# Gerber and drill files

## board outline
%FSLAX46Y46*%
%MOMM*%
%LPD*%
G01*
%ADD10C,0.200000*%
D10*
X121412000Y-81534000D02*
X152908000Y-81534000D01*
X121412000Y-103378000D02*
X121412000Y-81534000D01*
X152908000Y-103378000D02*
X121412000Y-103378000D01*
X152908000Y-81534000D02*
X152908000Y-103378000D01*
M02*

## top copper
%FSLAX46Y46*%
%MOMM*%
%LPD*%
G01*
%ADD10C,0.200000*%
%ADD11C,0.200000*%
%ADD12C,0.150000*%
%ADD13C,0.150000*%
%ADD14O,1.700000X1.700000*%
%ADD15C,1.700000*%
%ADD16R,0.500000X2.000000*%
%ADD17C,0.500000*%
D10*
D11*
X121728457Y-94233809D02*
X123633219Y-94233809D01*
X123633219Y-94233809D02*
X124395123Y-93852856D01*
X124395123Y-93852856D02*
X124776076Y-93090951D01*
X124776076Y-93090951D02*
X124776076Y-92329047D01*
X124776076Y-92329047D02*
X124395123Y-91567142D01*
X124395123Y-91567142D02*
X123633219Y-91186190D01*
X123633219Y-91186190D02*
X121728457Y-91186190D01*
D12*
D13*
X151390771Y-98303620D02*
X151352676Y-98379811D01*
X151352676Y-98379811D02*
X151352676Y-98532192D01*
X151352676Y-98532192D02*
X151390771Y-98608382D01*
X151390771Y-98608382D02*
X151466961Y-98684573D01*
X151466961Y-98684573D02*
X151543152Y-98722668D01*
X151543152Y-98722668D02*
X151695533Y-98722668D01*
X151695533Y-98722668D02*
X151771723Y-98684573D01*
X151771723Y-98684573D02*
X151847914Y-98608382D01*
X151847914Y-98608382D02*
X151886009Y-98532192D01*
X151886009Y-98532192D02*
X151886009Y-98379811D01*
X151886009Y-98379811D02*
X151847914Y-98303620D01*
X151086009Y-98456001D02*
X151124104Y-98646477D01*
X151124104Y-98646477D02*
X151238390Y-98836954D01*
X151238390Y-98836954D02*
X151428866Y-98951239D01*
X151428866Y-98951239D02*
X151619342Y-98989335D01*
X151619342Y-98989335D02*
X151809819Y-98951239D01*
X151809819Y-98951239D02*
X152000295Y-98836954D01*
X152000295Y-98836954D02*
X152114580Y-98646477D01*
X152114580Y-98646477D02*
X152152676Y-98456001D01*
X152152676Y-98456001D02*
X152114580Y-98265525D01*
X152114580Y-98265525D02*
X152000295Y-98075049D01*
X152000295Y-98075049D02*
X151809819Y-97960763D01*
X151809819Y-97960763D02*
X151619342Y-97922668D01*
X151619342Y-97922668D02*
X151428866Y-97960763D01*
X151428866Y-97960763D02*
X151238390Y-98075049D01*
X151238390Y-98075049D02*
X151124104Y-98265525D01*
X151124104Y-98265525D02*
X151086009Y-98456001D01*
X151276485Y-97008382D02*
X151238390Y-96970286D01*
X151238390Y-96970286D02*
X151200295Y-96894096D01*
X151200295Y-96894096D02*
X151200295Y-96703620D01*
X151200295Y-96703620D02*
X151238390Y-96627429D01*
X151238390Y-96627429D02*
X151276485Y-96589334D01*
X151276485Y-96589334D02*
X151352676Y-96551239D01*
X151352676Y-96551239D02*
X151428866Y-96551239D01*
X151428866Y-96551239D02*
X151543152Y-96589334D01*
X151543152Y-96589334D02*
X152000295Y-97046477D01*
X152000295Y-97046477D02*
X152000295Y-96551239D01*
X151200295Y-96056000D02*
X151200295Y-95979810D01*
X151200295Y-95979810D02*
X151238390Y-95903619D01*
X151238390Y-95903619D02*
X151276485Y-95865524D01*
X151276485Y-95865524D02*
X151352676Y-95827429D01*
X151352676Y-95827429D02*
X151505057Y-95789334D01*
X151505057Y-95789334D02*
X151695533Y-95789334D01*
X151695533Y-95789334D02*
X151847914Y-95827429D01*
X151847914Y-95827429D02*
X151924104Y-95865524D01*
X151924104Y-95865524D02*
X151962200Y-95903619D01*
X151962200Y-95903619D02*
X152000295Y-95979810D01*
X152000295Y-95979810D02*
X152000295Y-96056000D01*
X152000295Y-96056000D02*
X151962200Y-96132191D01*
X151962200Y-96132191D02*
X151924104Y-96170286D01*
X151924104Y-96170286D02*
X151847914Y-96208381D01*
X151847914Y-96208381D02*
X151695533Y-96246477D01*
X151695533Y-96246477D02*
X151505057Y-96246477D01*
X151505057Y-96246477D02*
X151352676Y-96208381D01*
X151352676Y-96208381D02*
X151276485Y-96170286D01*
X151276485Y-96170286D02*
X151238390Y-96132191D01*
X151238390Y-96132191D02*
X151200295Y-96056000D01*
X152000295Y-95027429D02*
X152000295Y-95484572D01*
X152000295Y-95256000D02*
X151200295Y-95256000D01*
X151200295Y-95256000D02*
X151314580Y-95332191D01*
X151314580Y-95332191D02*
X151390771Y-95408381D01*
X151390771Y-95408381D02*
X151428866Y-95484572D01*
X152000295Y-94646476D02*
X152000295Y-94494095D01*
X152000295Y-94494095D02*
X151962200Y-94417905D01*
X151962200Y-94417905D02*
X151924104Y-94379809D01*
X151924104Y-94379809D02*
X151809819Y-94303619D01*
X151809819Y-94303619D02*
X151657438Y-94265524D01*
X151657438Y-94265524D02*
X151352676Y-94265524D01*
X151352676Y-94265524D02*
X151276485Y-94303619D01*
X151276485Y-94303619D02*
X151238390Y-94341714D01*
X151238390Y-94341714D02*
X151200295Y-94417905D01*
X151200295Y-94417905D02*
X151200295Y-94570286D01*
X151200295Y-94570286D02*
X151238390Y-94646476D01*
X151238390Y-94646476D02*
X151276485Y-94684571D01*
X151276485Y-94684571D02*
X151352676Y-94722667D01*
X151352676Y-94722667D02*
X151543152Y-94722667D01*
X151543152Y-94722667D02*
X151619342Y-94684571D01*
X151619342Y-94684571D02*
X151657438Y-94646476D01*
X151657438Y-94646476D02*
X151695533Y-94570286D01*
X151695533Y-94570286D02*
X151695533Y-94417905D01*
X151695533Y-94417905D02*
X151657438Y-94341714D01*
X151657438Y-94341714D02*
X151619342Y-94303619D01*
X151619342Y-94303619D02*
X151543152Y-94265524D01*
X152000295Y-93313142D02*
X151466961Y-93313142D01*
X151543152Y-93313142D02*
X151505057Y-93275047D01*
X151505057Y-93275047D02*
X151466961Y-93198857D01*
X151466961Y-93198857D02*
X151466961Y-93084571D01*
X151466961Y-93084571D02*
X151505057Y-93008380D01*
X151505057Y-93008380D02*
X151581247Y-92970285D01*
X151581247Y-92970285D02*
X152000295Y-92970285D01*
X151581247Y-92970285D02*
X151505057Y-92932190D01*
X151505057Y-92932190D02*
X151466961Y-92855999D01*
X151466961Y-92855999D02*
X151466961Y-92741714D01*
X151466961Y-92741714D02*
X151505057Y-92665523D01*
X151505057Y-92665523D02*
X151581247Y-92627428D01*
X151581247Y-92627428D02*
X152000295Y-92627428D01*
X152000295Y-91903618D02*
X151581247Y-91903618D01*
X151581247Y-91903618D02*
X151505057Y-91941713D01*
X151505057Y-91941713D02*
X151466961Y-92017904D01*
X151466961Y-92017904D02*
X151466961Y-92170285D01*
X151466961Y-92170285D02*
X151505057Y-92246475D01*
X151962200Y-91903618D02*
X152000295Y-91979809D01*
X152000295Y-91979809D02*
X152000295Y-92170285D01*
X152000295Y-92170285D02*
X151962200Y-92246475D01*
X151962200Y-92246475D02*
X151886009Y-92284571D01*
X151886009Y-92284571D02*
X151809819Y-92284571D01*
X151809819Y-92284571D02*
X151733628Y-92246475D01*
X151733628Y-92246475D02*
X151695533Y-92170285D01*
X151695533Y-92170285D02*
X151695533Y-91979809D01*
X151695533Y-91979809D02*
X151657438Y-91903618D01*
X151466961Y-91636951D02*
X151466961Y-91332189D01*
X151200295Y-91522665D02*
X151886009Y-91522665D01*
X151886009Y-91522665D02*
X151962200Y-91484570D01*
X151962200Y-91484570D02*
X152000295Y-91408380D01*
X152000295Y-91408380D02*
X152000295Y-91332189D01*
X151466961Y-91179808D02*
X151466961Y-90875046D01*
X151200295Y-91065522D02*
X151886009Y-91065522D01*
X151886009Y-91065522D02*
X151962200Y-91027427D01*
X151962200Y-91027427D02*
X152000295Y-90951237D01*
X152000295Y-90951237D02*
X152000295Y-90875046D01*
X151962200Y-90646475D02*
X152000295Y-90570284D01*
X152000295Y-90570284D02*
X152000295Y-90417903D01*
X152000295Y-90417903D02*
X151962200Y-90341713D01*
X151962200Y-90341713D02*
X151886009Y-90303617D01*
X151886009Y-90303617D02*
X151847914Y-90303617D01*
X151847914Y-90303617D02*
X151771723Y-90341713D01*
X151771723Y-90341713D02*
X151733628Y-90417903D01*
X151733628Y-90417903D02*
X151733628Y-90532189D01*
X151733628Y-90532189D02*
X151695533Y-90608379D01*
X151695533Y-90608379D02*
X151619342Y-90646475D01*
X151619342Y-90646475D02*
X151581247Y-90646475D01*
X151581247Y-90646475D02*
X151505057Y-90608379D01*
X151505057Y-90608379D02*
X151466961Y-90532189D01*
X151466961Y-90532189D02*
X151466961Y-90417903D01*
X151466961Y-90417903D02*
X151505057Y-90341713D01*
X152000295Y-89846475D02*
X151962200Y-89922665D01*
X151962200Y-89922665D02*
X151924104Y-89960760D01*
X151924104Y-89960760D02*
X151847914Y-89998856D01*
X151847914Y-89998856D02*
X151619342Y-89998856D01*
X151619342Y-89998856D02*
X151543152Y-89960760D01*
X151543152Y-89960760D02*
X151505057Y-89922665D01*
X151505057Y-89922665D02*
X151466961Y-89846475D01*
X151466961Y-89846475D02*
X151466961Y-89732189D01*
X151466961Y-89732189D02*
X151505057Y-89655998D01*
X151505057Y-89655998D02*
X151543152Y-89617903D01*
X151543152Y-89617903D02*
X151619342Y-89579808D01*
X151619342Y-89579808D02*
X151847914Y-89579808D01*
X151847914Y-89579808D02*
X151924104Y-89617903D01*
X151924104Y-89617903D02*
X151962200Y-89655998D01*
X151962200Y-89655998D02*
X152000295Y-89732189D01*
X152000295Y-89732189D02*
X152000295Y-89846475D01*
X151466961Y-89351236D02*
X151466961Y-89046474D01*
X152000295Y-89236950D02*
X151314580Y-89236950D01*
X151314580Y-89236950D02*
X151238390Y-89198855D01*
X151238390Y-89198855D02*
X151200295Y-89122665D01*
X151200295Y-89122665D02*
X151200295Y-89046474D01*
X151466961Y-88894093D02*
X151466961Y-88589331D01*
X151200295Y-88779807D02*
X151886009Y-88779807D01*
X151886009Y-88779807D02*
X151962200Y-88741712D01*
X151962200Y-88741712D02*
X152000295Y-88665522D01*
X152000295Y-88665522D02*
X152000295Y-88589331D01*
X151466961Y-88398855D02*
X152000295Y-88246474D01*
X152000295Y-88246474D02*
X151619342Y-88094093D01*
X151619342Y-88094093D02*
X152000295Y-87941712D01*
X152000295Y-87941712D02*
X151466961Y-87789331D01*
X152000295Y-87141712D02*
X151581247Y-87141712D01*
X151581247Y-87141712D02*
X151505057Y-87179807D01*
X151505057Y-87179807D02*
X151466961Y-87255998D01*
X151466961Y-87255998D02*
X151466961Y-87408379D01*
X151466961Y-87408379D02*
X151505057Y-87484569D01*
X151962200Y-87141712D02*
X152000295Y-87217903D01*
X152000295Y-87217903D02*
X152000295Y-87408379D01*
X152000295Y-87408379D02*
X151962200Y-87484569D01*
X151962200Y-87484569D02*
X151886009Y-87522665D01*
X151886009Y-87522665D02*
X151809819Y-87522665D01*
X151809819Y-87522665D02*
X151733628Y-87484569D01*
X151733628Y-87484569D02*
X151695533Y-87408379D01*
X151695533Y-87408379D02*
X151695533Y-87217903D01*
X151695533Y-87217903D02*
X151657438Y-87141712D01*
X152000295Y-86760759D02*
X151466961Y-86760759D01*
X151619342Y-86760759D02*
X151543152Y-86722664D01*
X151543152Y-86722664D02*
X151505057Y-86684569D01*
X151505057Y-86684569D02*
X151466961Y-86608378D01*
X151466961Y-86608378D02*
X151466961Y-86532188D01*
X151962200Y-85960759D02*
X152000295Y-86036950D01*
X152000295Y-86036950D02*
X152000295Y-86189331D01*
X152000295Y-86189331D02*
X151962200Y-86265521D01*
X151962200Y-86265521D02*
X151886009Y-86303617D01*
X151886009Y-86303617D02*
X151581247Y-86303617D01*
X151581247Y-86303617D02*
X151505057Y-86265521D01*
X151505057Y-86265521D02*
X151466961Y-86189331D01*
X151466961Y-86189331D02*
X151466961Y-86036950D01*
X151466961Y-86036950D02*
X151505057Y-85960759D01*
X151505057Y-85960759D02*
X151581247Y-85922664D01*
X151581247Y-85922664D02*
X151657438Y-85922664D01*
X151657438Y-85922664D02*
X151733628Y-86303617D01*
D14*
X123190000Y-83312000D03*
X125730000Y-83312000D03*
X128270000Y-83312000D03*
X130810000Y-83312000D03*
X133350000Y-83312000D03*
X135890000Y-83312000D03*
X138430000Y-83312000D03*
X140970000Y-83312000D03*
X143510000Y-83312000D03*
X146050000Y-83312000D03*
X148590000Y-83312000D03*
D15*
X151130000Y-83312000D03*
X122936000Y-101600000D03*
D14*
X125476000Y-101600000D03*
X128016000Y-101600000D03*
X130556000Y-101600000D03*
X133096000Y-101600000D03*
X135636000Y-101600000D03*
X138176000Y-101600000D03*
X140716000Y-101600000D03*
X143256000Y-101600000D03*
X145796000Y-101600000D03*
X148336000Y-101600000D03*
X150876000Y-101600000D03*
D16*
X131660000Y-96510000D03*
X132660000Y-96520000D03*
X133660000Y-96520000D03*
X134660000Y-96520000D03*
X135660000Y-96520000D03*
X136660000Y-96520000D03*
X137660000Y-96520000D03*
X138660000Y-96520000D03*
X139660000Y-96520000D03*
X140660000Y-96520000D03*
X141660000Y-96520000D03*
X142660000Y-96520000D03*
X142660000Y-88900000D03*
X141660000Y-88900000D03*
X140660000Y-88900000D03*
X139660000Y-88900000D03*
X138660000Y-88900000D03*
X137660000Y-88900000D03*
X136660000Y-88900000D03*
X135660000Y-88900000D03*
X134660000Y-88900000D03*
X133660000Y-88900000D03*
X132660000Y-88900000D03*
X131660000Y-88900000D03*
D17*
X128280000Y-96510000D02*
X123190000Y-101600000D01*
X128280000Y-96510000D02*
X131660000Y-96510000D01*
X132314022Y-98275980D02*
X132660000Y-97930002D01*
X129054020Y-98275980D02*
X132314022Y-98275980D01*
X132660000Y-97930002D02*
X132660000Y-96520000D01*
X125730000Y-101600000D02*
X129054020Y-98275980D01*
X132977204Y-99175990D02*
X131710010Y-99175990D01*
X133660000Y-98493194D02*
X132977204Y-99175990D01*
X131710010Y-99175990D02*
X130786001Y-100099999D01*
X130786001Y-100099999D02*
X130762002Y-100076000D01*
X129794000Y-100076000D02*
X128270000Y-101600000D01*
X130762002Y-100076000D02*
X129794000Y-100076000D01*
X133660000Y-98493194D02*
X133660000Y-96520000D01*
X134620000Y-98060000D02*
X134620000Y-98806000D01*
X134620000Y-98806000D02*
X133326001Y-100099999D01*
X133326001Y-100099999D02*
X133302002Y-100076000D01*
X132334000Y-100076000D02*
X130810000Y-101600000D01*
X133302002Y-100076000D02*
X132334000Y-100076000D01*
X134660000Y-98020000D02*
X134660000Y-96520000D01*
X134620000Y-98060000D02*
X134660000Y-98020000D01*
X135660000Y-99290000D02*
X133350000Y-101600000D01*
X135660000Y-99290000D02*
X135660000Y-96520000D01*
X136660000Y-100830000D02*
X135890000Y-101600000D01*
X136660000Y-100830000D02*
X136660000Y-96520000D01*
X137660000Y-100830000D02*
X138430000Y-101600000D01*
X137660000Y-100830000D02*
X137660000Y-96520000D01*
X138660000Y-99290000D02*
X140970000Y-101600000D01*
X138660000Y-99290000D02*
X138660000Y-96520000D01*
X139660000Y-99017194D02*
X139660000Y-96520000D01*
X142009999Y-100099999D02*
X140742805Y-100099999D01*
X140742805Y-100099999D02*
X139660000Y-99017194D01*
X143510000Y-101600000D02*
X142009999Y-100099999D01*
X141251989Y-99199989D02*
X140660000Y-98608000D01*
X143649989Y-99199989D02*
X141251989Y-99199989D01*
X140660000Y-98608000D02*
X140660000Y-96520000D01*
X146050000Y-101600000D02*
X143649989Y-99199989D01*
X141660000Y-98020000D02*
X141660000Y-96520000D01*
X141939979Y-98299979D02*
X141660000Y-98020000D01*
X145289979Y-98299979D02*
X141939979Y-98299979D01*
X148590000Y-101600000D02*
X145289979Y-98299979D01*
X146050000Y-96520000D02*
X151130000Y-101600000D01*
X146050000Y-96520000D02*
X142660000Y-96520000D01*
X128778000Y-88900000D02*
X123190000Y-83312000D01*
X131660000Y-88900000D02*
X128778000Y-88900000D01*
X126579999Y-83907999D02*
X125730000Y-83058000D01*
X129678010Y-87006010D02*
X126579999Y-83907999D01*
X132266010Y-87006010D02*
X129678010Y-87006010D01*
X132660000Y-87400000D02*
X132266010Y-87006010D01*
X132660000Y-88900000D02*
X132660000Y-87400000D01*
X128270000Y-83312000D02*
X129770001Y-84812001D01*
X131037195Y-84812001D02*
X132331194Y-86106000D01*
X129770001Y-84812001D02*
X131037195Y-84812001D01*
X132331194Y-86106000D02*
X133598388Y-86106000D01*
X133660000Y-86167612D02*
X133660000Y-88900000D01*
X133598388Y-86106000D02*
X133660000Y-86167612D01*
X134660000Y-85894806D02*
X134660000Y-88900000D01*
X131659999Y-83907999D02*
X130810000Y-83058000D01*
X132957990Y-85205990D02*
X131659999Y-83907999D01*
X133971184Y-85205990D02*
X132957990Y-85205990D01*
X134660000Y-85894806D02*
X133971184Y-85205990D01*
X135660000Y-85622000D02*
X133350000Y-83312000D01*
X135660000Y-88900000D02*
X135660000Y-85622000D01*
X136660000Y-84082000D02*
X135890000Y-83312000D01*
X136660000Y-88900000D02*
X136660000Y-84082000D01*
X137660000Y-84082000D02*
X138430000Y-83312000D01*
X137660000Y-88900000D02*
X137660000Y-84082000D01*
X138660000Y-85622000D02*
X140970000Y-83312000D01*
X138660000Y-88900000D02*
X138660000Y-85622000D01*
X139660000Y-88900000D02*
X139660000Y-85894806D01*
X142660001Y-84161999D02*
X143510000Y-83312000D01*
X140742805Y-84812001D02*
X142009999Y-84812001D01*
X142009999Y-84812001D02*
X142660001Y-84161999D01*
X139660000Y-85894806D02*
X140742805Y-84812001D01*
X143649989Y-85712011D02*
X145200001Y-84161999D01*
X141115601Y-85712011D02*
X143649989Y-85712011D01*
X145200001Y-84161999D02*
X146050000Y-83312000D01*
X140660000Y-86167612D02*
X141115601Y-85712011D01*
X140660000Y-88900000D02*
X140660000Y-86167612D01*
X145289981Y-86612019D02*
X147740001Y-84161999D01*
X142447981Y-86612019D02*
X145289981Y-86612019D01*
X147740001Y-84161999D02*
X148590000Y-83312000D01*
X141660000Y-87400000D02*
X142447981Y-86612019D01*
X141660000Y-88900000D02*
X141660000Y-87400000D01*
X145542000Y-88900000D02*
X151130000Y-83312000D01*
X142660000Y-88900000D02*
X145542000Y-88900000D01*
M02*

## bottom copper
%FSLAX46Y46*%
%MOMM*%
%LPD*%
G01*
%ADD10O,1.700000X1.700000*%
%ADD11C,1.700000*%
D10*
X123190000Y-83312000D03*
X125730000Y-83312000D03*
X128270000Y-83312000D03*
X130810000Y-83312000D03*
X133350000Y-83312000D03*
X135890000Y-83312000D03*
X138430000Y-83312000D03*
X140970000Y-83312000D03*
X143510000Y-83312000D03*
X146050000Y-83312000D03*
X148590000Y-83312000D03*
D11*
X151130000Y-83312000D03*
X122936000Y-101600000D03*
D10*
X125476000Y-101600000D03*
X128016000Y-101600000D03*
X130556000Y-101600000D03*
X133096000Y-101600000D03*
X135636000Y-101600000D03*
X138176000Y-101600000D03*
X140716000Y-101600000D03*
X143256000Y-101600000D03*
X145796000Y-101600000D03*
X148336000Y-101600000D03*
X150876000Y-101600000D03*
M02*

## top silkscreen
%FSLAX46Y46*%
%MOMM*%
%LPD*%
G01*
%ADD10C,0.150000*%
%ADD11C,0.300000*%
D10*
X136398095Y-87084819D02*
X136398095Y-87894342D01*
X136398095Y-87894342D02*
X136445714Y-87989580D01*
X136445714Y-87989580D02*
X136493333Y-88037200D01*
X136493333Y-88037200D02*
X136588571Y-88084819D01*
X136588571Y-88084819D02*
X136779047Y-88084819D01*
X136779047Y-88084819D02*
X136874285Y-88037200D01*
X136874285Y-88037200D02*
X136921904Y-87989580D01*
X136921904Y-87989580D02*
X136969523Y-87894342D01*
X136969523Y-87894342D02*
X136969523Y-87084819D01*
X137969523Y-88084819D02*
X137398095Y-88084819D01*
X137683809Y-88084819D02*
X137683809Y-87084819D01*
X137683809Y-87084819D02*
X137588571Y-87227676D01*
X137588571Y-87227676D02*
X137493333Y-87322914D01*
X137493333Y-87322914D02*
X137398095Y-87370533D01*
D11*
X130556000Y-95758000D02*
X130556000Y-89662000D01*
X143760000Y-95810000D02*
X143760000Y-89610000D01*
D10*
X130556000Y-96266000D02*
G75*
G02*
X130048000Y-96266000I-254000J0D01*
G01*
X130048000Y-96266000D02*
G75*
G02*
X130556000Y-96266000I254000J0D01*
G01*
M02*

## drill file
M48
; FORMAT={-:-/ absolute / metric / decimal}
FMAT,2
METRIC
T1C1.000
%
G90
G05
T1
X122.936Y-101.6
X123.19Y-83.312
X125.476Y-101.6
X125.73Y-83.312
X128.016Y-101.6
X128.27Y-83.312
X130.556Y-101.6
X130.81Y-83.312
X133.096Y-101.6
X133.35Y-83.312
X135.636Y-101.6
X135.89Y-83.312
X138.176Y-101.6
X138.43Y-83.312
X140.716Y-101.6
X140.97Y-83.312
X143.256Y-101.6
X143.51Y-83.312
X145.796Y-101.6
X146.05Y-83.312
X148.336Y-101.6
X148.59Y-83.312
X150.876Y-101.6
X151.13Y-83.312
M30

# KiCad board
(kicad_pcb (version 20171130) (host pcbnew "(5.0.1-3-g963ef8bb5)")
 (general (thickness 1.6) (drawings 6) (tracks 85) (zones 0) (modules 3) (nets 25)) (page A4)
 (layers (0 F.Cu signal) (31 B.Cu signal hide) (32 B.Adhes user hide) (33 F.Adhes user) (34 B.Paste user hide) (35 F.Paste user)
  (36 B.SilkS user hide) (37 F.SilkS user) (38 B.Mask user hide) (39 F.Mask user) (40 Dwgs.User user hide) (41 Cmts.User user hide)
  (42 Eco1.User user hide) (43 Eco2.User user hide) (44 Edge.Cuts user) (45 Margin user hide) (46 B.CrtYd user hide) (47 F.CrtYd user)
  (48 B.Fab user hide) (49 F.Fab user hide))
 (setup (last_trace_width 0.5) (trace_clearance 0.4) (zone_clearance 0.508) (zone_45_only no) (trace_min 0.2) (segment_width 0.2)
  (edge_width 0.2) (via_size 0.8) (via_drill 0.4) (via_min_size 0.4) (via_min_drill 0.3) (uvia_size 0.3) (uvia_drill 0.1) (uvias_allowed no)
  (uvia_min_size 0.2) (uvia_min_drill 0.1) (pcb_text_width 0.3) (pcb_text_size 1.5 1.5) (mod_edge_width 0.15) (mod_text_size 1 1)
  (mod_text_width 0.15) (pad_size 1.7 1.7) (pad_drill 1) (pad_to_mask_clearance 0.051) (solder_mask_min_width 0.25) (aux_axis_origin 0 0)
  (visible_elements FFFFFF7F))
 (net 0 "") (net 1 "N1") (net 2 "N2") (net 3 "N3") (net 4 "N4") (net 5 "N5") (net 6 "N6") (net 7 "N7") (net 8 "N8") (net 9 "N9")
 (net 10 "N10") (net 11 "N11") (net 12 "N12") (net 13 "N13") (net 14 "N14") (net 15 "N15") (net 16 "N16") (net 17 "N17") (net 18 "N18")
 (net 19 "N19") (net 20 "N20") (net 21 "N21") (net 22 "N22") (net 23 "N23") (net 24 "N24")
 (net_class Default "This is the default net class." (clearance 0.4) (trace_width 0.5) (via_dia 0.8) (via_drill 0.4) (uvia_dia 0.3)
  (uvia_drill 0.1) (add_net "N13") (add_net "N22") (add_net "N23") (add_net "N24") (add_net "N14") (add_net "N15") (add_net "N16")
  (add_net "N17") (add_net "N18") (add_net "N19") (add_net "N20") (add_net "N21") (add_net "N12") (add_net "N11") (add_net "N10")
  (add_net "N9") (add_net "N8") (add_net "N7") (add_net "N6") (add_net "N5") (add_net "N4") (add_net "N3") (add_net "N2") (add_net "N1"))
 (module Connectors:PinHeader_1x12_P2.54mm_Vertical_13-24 (layer B.Cu) (at 151.13 83.312 90)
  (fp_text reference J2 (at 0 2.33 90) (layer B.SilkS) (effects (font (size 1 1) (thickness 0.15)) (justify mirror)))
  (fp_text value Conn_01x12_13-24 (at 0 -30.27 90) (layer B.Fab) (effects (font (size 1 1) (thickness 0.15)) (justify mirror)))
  (pad 24 thru_hole oval (at 0 -27.94 90) (size 1.7 1.7) (drill 1) (layers *.Cu *.Mask) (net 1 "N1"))
  (pad 23 thru_hole oval (at 0 -25.4 90) (size 1.7 1.7) (drill 1) (layers *.Cu *.Mask) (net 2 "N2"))
  (pad 22 thru_hole oval (at 0 -22.86 90) (size 1.7 1.7) (drill 1) (layers *.Cu *.Mask) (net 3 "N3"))
  (pad 21 thru_hole oval (at 0 -20.32 90) (size 1.7 1.7) (drill 1) (layers *.Cu *.Mask) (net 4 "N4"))
  (pad 20 thru_hole oval (at 0 -17.78 90) (size 1.7 1.7) (drill 1) (layers *.Cu *.Mask) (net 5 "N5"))
  (pad 19 thru_hole oval (at 0 -15.24 90) (size 1.7 1.7) (drill 1) (layers *.Cu *.Mask) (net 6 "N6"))
  (pad 18 thru_hole oval (at 0 -12.7 90) (size 1.7 1.7) (drill 1) (layers *.Cu *.Mask) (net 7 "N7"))
  (pad 17 thru_hole oval (at 0 -10.16 90) (size 1.7 1.7) (drill 1) (layers *.Cu *.Mask) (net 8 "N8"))
  (pad 16 thru_hole oval (at 0 -7.62 90) (size 1.7 1.7) (drill 1) (layers *.Cu *.Mask) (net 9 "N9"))
  (pad 15 thru_hole oval (at 0 -5.08 90) (size 1.7 1.7) (drill 1) (layers *.Cu *.Mask) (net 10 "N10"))
  (pad 14 thru_hole oval (at 0 -2.54 90) (size 1.7 1.7) (drill 1) (layers *.Cu *.Mask) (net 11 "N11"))
  (pad 13 thru_hole circle (at 0 0 90) (size 1.7 1.7) (drill 1) (layers *.Cu *.Mask) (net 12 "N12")))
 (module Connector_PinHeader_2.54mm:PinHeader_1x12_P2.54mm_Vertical (layer B.Cu) (at 122.936 101.6 270)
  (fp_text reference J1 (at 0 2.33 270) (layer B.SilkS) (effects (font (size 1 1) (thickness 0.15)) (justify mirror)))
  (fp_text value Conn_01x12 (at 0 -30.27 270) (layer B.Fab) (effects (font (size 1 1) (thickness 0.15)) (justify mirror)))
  (pad 1 thru_hole circle (at 0 0 270) (size 1.7 1.7) (drill 1) (layers *.Cu *.Mask) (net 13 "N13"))
  (pad 2 thru_hole oval (at 0 -2.54 270) (size 1.7 1.7) (drill 1) (layers *.Cu *.Mask) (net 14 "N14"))
  (pad 3 thru_hole oval (at 0 -5.08 270) (size 1.7 1.7) (drill 1) (layers *.Cu *.Mask) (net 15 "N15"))
  (pad 4 thru_hole oval (at 0 -7.62 270) (size 1.7 1.7) (drill 1) (layers *.Cu *.Mask) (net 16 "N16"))
  (pad 5 thru_hole oval (at 0 -10.16 270) (size 1.7 1.7) (drill 1) (layers *.Cu *.Mask) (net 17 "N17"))
  (pad 6 thru_hole oval (at 0 -12.7 270) (size 1.7 1.7) (drill 1) (layers *.Cu *.Mask) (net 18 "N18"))
  (pad 7 thru_hole oval (at 0 -15.24 270) (size 1.7 1.7) (drill 1) (layers *.Cu *.Mask) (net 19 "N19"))
  (pad 8 thru_hole oval (at 0 -17.78 270) (size 1.7 1.7) (drill 1) (layers *.Cu *.Mask) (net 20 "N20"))
  (pad 9 thru_hole oval (at 0 -20.32 270) (size 1.7 1.7) (drill 1) (layers *.Cu *.Mask) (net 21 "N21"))
  (pad 10 thru_hole oval (at 0 -22.86 270) (size 1.7 1.7) (drill 1) (layers *.Cu *.Mask) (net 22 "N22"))
  (pad 11 thru_hole oval (at 0 -25.4 270) (size 1.7 1.7) (drill 1) (layers *.Cu *.Mask) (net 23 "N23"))
  (pad 12 thru_hole oval (at 0 -27.94 270) (size 1.7 1.7) (drill 1) (layers *.Cu *.Mask) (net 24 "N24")))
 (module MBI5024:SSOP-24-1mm (layer F.Cu) (at 137.16 92.71)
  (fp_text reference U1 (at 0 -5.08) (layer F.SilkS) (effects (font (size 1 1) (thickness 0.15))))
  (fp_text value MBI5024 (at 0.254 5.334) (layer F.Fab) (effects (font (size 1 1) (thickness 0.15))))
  (fp_line (start -6.604 3.048) (end -6.604 -3.048) (layer F.SilkS) (width 0.3))
  (fp_line (start 6.6 3.1) (end 6.6 -3.1) (layer F.SilkS) (width 0.3))
  (fp_circle (center -6.858 3.556) (end -6.858 3.302) (layer F.SilkS) (width 0.15))
  (pad 1 smd rect (at -5.5 3.8) (size 0.5 2) (layers F.Cu F.Paste F.Mask) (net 13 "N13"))
  (pad 2 smd rect (at -4.5 3.81) (size 0.5 2) (layers F.Cu F.Paste F.Mask) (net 14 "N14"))
  (pad 3 smd rect (at -3.5 3.81) (size 0.5 2) (layers F.Cu F.Paste F.Mask) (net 15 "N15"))
  (pad 4 smd rect (at -2.5 3.81) (size 0.5 2) (layers F.Cu F.Paste F.Mask) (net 16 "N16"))
  (pad 5 smd rect (at -1.5 3.81) (size 0.5 2) (layers F.Cu F.Paste F.Mask) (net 17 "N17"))
  (pad 6 smd rect (at -0.5 3.81) (size 0.5 2) (layers F.Cu F.Paste F.Mask) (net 18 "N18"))
  (pad 7 smd rect (at 0.5 3.81) (size 0.5 2) (layers F.Cu F.Paste F.Mask) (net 19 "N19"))
  (pad 8 smd rect (at 1.5 3.81) (size 0.5 2) (layers F.Cu F.Paste F.Mask) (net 20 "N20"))
  (pad 9 smd rect (at 2.5 3.81) (size 0.5 2) (layers F.Cu F.Paste F.Mask) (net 21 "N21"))
  (pad 10 smd rect (at 3.5 3.81) (size 0.5 2) (layers F.Cu F.Paste F.Mask) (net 22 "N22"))
  (pad 11 smd rect (at 4.5 3.81) (size 0.5 2) (layers F.Cu F.Paste F.Mask) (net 23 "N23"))
  (pad 12 smd rect (at 5.5 3.81) (size 0.5 2) (layers F.Cu F.Paste F.Mask) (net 24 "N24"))
  (pad 13 smd rect (at 5.5 -3.81) (size 0.5 2) (layers F.Cu F.Paste F.Mask) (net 12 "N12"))
  (pad 14 smd rect (at 4.5 -3.81) (size 0.5 2) (layers F.Cu F.Paste F.Mask) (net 11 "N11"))
  (pad 15 smd rect (at 3.5 -3.81) (size 0.5 2) (layers F.Cu F.Paste F.Mask) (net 10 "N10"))
  (pad 16 smd rect (at 2.5 -3.81) (size 0.5 2) (layers F.Cu F.Paste F.Mask) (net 9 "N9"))
  (pad 17 smd rect (at 1.5 -3.81) (size 0.5 2) (layers F.Cu F.Paste F.Mask) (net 8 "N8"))
  (pad 18 smd rect (at 0.5 -3.81) (size 0.5 2) (layers F.Cu F.Paste F.Mask) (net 7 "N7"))
  (pad 19 smd rect (at -0.5 -3.81) (size 0.5 2) (layers F.Cu F.Paste F.Mask) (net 6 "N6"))
  (pad 20 smd rect (at -1.5 -3.81) (size 0.5 2) (layers F.Cu F.Paste F.Mask) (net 5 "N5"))
  (pad 21 smd rect (at -2.5 -3.81) (size 0.5 2) (layers F.Cu F.Paste F.Mask) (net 4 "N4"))
  (pad 22 smd rect (at -3.5 -3.81) (size 0.5 2) (layers F.Cu F.Paste F.Mask) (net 3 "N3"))
  (pad 23 smd rect (at -4.5 -3.81) (size 0.5 2) (layers F.Cu F.Paste F.Mask) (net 2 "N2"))
  (pad 24 smd rect (at -5.5 -3.81) (size 0.5 2) (layers F.Cu F.Paste F.Mask) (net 1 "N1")))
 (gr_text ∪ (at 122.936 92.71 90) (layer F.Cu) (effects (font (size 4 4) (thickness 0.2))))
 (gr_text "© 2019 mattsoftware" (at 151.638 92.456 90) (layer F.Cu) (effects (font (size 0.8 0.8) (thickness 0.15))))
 (gr_line (start 121.412 81.534) (end 152.908 81.534) (layer Edge.Cuts) (width 0.2))
 (gr_line (start 121.412 103.378) (end 121.412 81.534) (layer Edge.Cuts) (width 0.2))
 (gr_line (start 152.908 103.378) (end 121.412 103.378) (layer Edge.Cuts) (width 0.2))
 (gr_line (start 152.908 81.534) (end 152.908 103.378) (layer Edge.Cuts) (width 0.2))
 (segment (start 128.28 96.51) (end 123.19 101.6) (width 0.5) (layer F.Cu) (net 13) (status 20))
 (segment (start 128.28 96.51) (end 131.66 96.51) (width 0.5) (layer F.Cu) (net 13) (status 20))
 (segment (start 132.314022 98.27598) (end 132.66 97.930002) (width 0.5) (layer F.Cu) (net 14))
 (segment (start 129.05402 98.27598) (end 132.314022 98.27598) (width 0.5) (layer F.Cu) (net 14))
 (segment (start 132.66 97.930002) (end 132.66 96.52) (width 0.5) (layer F.Cu) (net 14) (status 20))
 (segment (start 125.73 101.6) (end 129.05402 98.27598) (width 0.5) (layer F.Cu) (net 14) (status 10))
 (segment (start 132.977204 99.17599) (end 131.71001 99.17599) (width 0.5) (layer F.Cu) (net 15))
 (segment (start 133.66 98.493194) (end 132.977204 99.17599) (width 0.5) (layer F.Cu) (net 15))
 (segment (start 131.71001 99.17599) (end 130.786001 100.099999) (width 0.5) (layer F.Cu) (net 15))
 (segment (start 130.786001 100.099999) (end 130.762002 100.076) (width 0.5) (layer F.Cu) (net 15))
 (segment (start 129.794 100.076) (end 128.27 101.6) (width 0.5) (layer F.Cu) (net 15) (status 20))
 (segment (start 130.762002 100.076) (end 129.794 100.076) (width 0.5) (layer F.Cu) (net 15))
 (segment (start 133.66 98.493194) (end 133.66 96.52) (width 0.5) (layer F.Cu) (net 15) (status 20))
 (segment (start 134.62 98.06) (end 134.62 98.806) (width 0.5) (layer F.Cu) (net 16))
 (segment (start 134.62 98.806) (end 133.326001 100.099999) (width 0.5) (layer F.Cu) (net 16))
 (segment (start 133.326001 100.099999) (end 133.302002 100.076) (width 0.5) (layer F.Cu) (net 16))
 (segment (start 132.334 100.076) (end 130.81 101.6) (width 0.5) (layer F.Cu) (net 16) (status 20))
 (segment (start 133.302002 100.076) (end 132.334 100.076) (width 0.5) (layer F.Cu) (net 16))
 (segment (start 134.66 98.02) (end 134.66 96.52) (width 0.5) (layer F.Cu) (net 16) (status 20))
 (segment (start 134.62 98.06) (end 134.66 98.02) (width 0.5) (layer F.Cu) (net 16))
 (segment (start 135.66 99.29) (end 133.35 101.6) (width 0.5) (layer F.Cu) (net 17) (status 20))
 (segment (start 135.66 99.29) (end 135.66 96.52) (width 0.5) (layer F.Cu) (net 17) (status 20))
 (segment (start 136.66 100.83) (end 135.89 101.6) (width 0.5) (layer F.Cu) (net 18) (status 20))
 (segment (start 136.66 100.83) (end 136.66 96.52) (width 0.5) (layer F.Cu) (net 18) (status 20))
 (segment (start 137.66 100.83) (end 138.43 101.6) (width 0.5) (layer F.Cu) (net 19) (status 30))
 (segment (start 137.66 100.83) (end 137.66 96.52) (width 0.5) (layer F.Cu) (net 19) (status 30))
 (segment (start 138.66 99.29) (end 140.97 101.6) (width 0.5) (layer F.Cu) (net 20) (status 20))
 (segment (start 138.66 99.29) (end 138.66 96.52) (width 0.5) (layer F.Cu) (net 20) (status 20))
 (segment (start 139.66 99.017194) (end 139.66 96.52) (width 0.5) (layer F.Cu) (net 21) (status 20))
 (segment (start 142.009999 100.099999) (end 140.742805 100.099999) (width 0.5) (layer F.Cu) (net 21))
 (segment (start 140.742805 100.099999) (end 139.66 99.017194) (width 0.5) (layer F.Cu) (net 21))
 (segment (start 143.51 101.6) (end 142.009999 100.099999) (width 0.5) (layer F.Cu) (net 21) (status 10))
 (segment (start 141.251989 99.199989) (end 140.66 98.608) (width 0.5) (layer F.Cu) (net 22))
 (segment (start 143.649989 99.199989) (end 141.251989 99.199989) (width 0.5) (layer F.Cu) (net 22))
 (segment (start 140.66 98.608) (end 140.66 96.52) (width 0.5) (layer F.Cu) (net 22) (status 20))
 (segment (start 146.05 101.6) (end 143.649989 99.199989) (width 0.5) (layer F.Cu) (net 22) (status 10))
 (segment (start 141.66 98.02) (end 141.66 96.52) (width 0.5) (layer F.Cu) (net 23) (status 20))
 (segment (start 141.939979 98.299979) (end 141.66 98.02) (width 0.5) (layer F.Cu) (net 23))
 (segment (start 145.289979 98.299979) (end 141.939979 98.299979) (width 0.5) (layer F.Cu) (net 23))
 (segment (start 148.59 101.6) (end 145.289979 98.299979) (width 0.5) (layer F.Cu) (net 23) (status 10))
 (segment (start 146.05 96.52) (end 151.13 101.6) (width 0.5) (layer F.Cu) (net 24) (status 20))
 (segment (start 146.05 96.52) (end 142.66 96.52) (width 0.5) (layer F.Cu) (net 24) (status 20))
 (segment (start 128.778 88.9) (end 123.19 83.312) (width 0.5) (layer F.Cu) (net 1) (status 20))
 (segment (start 131.66 88.9) (end 128.778 88.9) (width 0.5) (layer F.Cu) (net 1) (status 10))
 (segment (start 126.579999 83.907999) (end 125.73 83.058) (width 0.5) (layer F.Cu) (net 2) (status 30))
 (segment (start 129.67801 87.00601) (end 126.579999 83.907999) (width 0.5) (layer F.Cu) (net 2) (status 20))
 (segment (start 132.26601 87.00601) (end 129.67801 87.00601) (width 0.5) (layer F.Cu) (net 2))
 (segment (start 132.66 87.4) (end 132.26601 87.00601) (width 0.5) (layer F.Cu) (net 2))
 (segment (start 132.66 88.9) (end 132.66 87.4) (width 0.5) (layer F.Cu) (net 2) (status 10))
 (segment (start 128.27 83.312) (end 129.770001 84.812001) (width 0.5) (layer F.Cu) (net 3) (status 10))
 (segment (start 131.037195 84.812001) (end 132.331194 86.106) (width 0.5) (layer F.Cu) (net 3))
 (segment (start 129.770001 84.812001) (end 131.037195 84.812001) (width 0.5) (layer F.Cu) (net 3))
 (segment (start 132.331194 86.106) (end 133.598388 86.106) (width 0.5) (layer F.Cu) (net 3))
 (segment (start 133.66 86.167612) (end 133.66 88.9) (width 0.5) (layer F.Cu) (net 3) (status 20))
 (segment (start 133.598388 86.106) (end 133.66 86.167612) (width 0.5) (layer F.Cu) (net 3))
 (segment (start 134.66 85.894806) (end 134.66 88.9) (width 0.5) (layer F.Cu) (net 4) (status 20))
 (segment (start 131.659999 83.907999) (end 130.81 83.058) (width 0.5) (layer F.Cu) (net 4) (status 30))
 (segment (start 132.95799 85.20599) (end 131.659999 83.907999) (width 0.5) (layer F.Cu) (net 4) (status 20))
 (segment (start 133.971184 85.20599) (end 132.95799 85.20599) (width 0.5) (layer F.Cu) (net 4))
 (segment (start 134.66 85.894806) (end 133.971184 85.20599) (width 0.5) (layer F.Cu) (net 4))
 (segment (start 135.66 85.622) (end 133.35 83.312) (width 0.5) (layer F.Cu) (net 5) (status 20))
 (segment (start 135.66 88.9) (end 135.66 85.622) (width 0.5) (layer F.Cu) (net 5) (status 10))
 (segment (start 136.66 84.082) (end 135.89 83.312) (width 0.5) (layer F.Cu) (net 6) (status 30))
 (segment (start 136.66 88.9) (end 136.66 84.082) (width 0.5) (layer F.Cu) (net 6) (status 30))
 (segment (start 137.66 84.082) (end 138.43 83.312) (width 0.5) (layer F.Cu) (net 7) (status 30))
 (segment (start 137.66 88.9) (end 137.66 84.082) (width 0.5) (layer F.Cu) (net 7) (status 30))
 (segment (start 138.66 85.622) (end 140.97 83.312) (width 0.5) (layer F.Cu) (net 8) (status 20))
 (segment (start 138.66 88.9) (end 138.66 85.622) (width 0.5) (layer F.Cu) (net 8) (status 10))
 (segment (start 139.66 88.9) (end 139.66 85.894806) (width 0.5) (layer F.Cu) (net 9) (status 10))
 (segment (start 142.660001 84.161999) (end 143.51 83.312) (width 0.5) (layer F.Cu) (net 9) (status 30))
 (segment (start 140.742805 84.812001) (end 142.009999 84.812001) (width 0.5) (layer F.Cu) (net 9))
 (segment (start 142.009999 84.812001) (end 142.660001 84.161999) (width 0.5) (layer F.Cu) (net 9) (status 20))
 (segment (start 139.66 85.894806) (end 140.742805 84.812001) (width 0.5) (layer F.Cu) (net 9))
 (segment (start 143.649989 85.712011) (end 145.200001 84.161999) (width 0.5) (layer F.Cu) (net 10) (status 20))
 (segment (start 141.115601 85.712011) (end 143.649989 85.712011) (width 0.5) (layer F.Cu) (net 10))
 (segment (start 145.200001 84.161999) (end 146.05 83.312) (width 0.5) (layer F.Cu) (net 10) (status 30))
 (segment (start 140.66 86.167612) (end 141.115601 85.712011) (width 0.5) (layer F.Cu) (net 10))
 (segment (start 140.66 88.9) (end 140.66 86.167612) (width 0.5) (layer F.Cu) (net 10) (status 10))
 (segment (start 145.289981 86.612019) (end 147.740001 84.161999) (width 0.5) (layer F.Cu) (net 11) (status 20))
 (segment (start 142.447981 86.612019) (end 145.289981 86.612019) (width 0.5) (layer F.Cu) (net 11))
 (segment (start 147.740001 84.161999) (end 148.59 83.312) (width 0.5) (layer F.Cu) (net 11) (status 30))
 (segment (start 141.66 87.4) (end 142.447981 86.612019) (width 0.5) (layer F.Cu) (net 11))
 (segment (start 141.66 88.9) (end 141.66 87.4) (width 0.5) (layer F.Cu) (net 11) (status 10))
 (segment (start 145.542 88.9) (end 151.13 83.312) (width 0.5) (layer F.Cu) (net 12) (status 20))
 (segment (start 142.66 88.9) (end 145.542 88.9) (width 0.5) (layer F.Cu) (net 12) (status 10)))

